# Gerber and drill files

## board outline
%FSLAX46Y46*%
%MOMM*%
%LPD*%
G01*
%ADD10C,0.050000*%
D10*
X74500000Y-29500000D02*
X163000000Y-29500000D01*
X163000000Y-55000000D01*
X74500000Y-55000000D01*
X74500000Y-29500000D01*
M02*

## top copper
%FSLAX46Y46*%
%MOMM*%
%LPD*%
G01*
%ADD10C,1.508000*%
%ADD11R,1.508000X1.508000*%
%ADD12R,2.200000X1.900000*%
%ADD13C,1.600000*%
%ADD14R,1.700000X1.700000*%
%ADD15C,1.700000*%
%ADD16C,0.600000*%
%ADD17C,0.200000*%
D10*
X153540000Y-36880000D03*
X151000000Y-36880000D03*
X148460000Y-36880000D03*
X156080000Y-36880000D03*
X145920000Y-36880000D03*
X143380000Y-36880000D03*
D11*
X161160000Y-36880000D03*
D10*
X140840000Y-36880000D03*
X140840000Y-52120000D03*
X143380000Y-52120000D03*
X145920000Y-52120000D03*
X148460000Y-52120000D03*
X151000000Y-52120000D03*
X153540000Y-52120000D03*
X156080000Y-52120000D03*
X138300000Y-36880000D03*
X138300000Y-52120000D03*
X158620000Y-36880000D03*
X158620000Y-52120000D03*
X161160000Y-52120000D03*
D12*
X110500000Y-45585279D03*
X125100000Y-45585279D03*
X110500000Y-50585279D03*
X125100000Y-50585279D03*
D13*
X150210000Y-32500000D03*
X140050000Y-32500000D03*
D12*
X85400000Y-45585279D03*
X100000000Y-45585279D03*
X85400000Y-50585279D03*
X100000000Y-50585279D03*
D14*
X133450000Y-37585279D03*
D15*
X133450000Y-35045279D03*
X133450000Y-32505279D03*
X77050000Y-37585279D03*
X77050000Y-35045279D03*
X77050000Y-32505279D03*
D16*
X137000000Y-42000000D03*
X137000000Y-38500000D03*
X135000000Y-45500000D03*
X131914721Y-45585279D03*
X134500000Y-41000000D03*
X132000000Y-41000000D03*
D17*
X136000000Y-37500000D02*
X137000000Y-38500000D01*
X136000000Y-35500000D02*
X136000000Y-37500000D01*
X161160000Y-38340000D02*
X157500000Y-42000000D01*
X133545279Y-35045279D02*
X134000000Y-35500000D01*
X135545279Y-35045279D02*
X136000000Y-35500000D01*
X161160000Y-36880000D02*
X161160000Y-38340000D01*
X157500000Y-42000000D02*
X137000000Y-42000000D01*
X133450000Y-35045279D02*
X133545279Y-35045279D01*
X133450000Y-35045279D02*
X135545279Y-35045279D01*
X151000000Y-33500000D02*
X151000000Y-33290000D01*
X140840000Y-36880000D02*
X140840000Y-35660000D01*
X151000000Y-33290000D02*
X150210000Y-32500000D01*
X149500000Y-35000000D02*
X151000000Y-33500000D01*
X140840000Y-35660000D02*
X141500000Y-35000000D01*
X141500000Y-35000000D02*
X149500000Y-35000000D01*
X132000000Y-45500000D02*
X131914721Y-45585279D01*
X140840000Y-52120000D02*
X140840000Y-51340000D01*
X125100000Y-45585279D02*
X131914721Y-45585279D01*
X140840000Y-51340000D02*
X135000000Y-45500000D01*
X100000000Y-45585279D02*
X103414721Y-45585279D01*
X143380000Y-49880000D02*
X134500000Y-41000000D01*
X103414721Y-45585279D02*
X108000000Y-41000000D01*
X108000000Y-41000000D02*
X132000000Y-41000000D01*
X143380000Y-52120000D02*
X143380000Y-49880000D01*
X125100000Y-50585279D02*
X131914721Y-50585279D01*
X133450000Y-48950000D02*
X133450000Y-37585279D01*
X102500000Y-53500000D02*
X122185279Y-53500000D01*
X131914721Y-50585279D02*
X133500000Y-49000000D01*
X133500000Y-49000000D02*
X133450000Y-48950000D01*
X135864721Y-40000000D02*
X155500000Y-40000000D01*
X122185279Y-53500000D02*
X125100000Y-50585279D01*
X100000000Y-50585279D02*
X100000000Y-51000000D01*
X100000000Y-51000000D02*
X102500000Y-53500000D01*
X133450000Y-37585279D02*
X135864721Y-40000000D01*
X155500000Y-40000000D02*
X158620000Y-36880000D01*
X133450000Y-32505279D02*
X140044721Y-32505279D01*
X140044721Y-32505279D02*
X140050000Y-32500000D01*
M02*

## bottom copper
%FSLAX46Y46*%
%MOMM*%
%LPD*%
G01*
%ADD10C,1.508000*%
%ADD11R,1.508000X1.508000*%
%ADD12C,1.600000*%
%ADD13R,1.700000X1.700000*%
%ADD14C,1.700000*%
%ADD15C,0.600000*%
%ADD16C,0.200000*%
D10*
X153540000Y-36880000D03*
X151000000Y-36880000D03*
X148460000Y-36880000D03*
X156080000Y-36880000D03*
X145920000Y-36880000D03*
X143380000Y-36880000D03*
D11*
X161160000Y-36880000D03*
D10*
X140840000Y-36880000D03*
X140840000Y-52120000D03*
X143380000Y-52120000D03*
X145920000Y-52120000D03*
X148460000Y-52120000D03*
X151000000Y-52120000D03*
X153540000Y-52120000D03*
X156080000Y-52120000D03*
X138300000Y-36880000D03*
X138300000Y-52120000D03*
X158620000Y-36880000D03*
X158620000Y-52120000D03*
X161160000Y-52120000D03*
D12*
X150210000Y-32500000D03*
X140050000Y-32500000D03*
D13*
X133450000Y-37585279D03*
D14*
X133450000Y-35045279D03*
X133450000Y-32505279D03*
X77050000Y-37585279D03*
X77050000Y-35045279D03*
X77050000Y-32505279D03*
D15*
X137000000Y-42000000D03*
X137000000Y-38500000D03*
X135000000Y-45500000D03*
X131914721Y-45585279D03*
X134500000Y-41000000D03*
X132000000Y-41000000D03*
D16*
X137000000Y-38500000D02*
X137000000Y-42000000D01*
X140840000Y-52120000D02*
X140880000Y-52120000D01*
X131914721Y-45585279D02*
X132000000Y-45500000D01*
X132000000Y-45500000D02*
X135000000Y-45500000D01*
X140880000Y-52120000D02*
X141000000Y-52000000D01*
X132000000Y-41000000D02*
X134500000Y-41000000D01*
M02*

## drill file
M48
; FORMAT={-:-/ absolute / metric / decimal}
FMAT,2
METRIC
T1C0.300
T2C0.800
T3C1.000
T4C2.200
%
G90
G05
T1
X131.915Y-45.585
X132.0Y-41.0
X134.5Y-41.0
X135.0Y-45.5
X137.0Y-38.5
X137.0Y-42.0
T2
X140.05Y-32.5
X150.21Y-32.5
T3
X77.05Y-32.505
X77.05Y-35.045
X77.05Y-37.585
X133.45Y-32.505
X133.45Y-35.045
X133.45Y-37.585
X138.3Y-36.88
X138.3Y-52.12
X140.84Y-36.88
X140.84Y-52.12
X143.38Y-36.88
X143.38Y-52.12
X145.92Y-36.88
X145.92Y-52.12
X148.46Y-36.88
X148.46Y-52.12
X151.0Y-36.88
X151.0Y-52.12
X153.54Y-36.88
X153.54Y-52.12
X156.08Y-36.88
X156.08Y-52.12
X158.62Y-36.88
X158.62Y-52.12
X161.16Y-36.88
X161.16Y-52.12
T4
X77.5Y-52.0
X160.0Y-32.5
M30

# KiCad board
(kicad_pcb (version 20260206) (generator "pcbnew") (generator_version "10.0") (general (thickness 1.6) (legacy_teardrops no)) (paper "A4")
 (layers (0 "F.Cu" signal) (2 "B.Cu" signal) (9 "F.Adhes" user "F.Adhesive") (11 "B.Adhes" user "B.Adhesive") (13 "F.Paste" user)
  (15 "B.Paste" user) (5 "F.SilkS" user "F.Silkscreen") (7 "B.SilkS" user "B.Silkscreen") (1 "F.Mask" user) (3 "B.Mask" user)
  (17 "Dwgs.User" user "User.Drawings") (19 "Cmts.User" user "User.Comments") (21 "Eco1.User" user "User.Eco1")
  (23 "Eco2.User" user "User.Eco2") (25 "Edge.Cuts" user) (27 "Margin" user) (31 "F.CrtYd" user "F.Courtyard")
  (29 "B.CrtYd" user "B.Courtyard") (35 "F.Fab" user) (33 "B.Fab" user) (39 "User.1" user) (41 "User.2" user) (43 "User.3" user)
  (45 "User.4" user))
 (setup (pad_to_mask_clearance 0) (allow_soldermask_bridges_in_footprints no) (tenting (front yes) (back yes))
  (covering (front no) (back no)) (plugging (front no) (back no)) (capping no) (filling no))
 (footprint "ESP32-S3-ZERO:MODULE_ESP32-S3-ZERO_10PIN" (layer "F.Cu") (at 151 44.5 -90)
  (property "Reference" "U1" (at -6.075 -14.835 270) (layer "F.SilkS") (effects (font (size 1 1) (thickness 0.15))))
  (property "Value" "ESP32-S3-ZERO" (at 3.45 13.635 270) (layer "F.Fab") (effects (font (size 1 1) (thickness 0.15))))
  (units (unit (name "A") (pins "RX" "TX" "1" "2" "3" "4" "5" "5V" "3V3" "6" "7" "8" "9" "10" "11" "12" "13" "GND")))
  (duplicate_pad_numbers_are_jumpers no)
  (pad "1" thru_hole circle (at -7.62 -2.54 270) (size 1.508 1.508) (drill 1) (layers "*.Cu" "*.Mask") (remove_unused_layers no)
   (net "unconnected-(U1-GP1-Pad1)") (solder_mask_margin 0.102))
  (pad "2" thru_hole circle (at -7.62 0 270) (size 1.508 1.508) (drill 1) (layers "*.Cu" "*.Mask") (remove_unused_layers no)
   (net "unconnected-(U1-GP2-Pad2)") (solder_mask_margin 0.102))
  (pad "3" thru_hole circle (at -7.62 2.54 270) (size 1.508 1.508) (drill 1) (layers "*.Cu" "*.Mask") (remove_unused_layers no)
   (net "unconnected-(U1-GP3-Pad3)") (solder_mask_margin 0.102))
  (pad "3V3" thru_hole circle (at -7.62 -5.08 270) (size 1.508 1.508) (drill 1) (layers "*.Cu" "*.Mask") (remove_unused_layers no)
   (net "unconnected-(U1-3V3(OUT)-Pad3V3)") (solder_mask_margin 0.102))
  (pad "4" thru_hole circle (at -7.62 5.08 270) (size 1.508 1.508) (drill 1) (layers "*.Cu" "*.Mask") (remove_unused_layers no)
   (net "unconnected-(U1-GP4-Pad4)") (solder_mask_margin 0.102))
  (pad "5" thru_hole circle (at -7.62 7.62 270) (size 1.508 1.508) (drill 1) (layers "*.Cu" "*.Mask") (remove_unused_layers no)
   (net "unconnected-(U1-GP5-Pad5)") (solder_mask_margin 0.102))
  (pad "5V" thru_hole rect (at -7.62 -10.16 270) (size 1.508 1.508) (drill 1) (layers "*.Cu" "*.Mask") (remove_unused_layers no)
   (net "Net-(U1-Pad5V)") (solder_mask_margin 0.102))
  (pad "6" thru_hole circle (at -7.62 10.16 270) (size 1.508 1.508) (drill 1) (layers "*.Cu" "*.Mask") (remove_unused_layers no)
   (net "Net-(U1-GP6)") (solder_mask_margin 0.102))
  (pad "7" thru_hole circle (at 7.62 10.16 270) (size 1.508 1.508) (drill 1) (layers "*.Cu" "*.Mask") (remove_unused_layers no)
   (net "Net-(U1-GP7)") (solder_mask_margin 0.102))
  (pad "8" thru_hole circle (at 7.62 7.62 270) (size 1.508 1.508) (drill 1) (layers "*.Cu" "*.Mask") (remove_unused_layers no)
   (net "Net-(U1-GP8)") (solder_mask_margin 0.102))
  (pad "9" thru_hole circle (at 7.62 5.08 270) (size 1.508 1.508) (drill 1) (layers "*.Cu" "*.Mask") (remove_unused_layers no)
   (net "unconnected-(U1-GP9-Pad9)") (solder_mask_margin 0.102))
  (pad "10" thru_hole circle (at 7.62 2.54 270) (size 1.508 1.508) (drill 1) (layers "*.Cu" "*.Mask") (remove_unused_layers no)
   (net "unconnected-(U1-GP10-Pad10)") (solder_mask_margin 0.102))
  (pad "11" thru_hole circle (at 7.62 0 270) (size 1.508 1.508) (drill 1) (layers "*.Cu" "*.Mask") (remove_unused_layers no)
   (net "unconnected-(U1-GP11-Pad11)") (solder_mask_margin 0.102))
  (pad "12" thru_hole circle (at 7.62 -2.54 270) (size 1.508 1.508) (drill 1) (layers "*.Cu" "*.Mask") (remove_unused_layers no)
   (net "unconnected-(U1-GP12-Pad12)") (solder_mask_margin 0.102))
  (pad "13" thru_hole circle (at 7.62 -5.08 270) (size 1.508 1.508) (drill 1) (layers "*.Cu" "*.Mask") (remove_unused_layers no)
   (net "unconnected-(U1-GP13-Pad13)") (solder_mask_margin 0.102))
  (pad "14" thru_hole circle (at -7.62 12.7 270) (size 1.508 1.508) (drill 1) (layers "*.Cu" "*.Mask") (remove_unused_layers no)
   (solder_mask_margin 0.102))
  (pad "15" thru_hole circle (at 7.62 12.7 270) (size 1.508 1.508) (drill 1) (layers "*.Cu" "*.Mask") (remove_unused_layers no)
   (solder_mask_margin 0.102))
  (pad "GND" thru_hole circle (at -7.62 -7.62 270) (size 1.508 1.508) (drill 1) (layers "*.Cu" "*.Mask") (remove_unused_layers no)
   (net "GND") (solder_mask_margin 0.102))
  (pad "RX" thru_hole circle (at 7.62 -7.62 270) (size 1.508 1.508) (drill 1) (layers "*.Cu" "*.Mask") (remove_unused_layers no)
   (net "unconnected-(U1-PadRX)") (solder_mask_margin 0.102))
  (pad "TX" thru_hole circle (at 7.62 -10.16 270) (size 1.508 1.508) (drill 1) (layers "*.Cu" "*.Mask") (remove_unused_layers no)
   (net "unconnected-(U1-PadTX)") (solder_mask_margin 0.102)))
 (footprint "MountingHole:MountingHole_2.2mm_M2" (layer "F.Cu") (at 77.5 52)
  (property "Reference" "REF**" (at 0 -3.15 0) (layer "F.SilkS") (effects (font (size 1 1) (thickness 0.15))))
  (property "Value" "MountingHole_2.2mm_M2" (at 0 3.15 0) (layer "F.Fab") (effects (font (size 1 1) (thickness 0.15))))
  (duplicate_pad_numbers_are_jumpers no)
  (pad "" np_thru_hole circle (at 0 0) (size 2.2 2.2) (drill 2.2) (layers "*.Cu" "*.Mask")))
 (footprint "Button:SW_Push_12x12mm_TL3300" (layer "F.Cu") (at 117.8 48.085279)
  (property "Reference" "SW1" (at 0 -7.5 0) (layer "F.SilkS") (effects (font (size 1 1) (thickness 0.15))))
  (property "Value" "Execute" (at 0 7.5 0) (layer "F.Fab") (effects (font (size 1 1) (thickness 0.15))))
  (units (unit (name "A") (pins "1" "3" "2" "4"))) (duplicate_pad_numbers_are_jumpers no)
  (pad "1" smd rect (at -7.3 -2.5) (size 2.2 1.9) (layers "F.Cu" "F.Mask" "F.Paste") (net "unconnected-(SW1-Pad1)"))
  (pad "2" smd rect (at 7.3 -2.5) (size 2.2 1.9) (layers "F.Cu" "F.Mask" "F.Paste") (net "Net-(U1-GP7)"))
  (pad "3" smd rect (at -7.3 2.5) (size 2.2 1.9) (layers "F.Cu" "F.Mask" "F.Paste") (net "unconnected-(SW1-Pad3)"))
  (pad "4" smd rect (at 7.3 2.5) (size 2.2 1.9) (layers "F.Cu" "F.Mask" "F.Paste") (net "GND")))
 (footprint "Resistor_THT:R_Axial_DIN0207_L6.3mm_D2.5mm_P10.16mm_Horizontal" (layer "F.Cu") (at 150.21 32.5 180)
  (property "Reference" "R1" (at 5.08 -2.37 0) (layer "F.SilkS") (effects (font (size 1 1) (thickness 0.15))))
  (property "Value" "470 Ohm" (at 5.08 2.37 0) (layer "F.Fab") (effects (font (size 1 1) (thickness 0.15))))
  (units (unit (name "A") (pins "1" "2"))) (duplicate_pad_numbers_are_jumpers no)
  (pad "1" thru_hole circle (at 0 0 180) (size 1.6 1.6) (drill 0.8) (layers "*.Cu" "*.Mask") (remove_unused_layers no) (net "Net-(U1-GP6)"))
  (pad "2" thru_hole circle (at 10.16 0 180) (size 1.6 1.6) (drill 0.8) (layers "*.Cu" "*.Mask") (remove_unused_layers no)
   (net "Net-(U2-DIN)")))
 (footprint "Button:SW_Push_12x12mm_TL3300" (layer "F.Cu") (at 92.7 48.085279)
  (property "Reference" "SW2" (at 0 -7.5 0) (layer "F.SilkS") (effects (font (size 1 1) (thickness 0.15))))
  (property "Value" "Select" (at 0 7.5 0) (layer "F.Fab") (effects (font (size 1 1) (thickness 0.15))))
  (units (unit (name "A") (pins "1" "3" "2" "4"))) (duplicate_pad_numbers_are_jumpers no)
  (pad "1" smd rect (at -7.3 -2.5) (size 2.2 1.9) (layers "F.Cu" "F.Mask" "F.Paste") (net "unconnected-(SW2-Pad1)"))
  (pad "2" smd rect (at 7.3 -2.5) (size 2.2 1.9) (layers "F.Cu" "F.Mask" "F.Paste") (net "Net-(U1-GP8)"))
  (pad "3" smd rect (at -7.3 2.5) (size 2.2 1.9) (layers "F.Cu" "F.Mask" "F.Paste") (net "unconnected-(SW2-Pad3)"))
  (pad "4" smd rect (at 7.3 2.5) (size 2.2 1.9) (layers "F.Cu" "F.Mask" "F.Paste") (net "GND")))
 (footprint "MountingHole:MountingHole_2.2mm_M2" (layer "F.Cu") (at 160 32.5)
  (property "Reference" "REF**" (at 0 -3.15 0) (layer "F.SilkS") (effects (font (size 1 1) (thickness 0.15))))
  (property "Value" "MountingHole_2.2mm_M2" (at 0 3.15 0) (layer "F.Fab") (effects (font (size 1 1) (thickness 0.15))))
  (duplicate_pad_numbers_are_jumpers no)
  (pad "" np_thru_hole circle (at 0 0) (size 2.2 2.2) (drill 2.2) (layers "*.Cu" "*.Mask")))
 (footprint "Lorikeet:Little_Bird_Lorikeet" (layer "F.Cu") (at 105.25 35.045279 180)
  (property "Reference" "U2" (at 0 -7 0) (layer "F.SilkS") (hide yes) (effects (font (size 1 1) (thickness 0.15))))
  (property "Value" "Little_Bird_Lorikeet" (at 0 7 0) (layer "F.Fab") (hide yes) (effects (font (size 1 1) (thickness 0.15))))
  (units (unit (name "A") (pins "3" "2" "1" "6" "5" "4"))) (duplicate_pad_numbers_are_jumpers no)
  (pad "1" thru_hole rect (at -28.2 -2.54 180) (size 1.7 1.7) (drill 1) (layers "*.Cu" "*.Mask") (remove_unused_layers no) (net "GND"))
  (pad "2" thru_hole circle (at -28.2 0 180) (size 1.7 1.7) (drill 1) (layers "*.Cu" "*.Mask") (remove_unused_layers no)
   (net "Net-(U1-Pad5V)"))
  (pad "3" thru_hole circle (at -28.2 2.54 180) (size 1.7 1.7) (drill 1) (layers "*.Cu" "*.Mask") (remove_unused_layers no)
   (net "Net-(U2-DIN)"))
  (pad "4" thru_hole circle (at 28.2 -2.54 180) (size 1.7 1.7) (drill 1) (layers "*.Cu" "*.Mask") (remove_unused_layers no)
   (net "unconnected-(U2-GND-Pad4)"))
  (pad "5" thru_hole circle (at 28.2 0 180) (size 1.7 1.7) (drill 1) (layers "*.Cu" "*.Mask") (remove_unused_layers no)
   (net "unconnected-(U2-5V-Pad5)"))
  (pad "6" thru_hole circle (at 28.2 2.54 180) (size 1.7 1.7) (drill 1) (layers "*.Cu" "*.Mask") (remove_unused_layers no)
   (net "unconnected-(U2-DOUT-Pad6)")))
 (gr_rect (start 74.5 29.5) (end 163 55) (stroke (width 0.05) (type default)) (fill no) (layer "Edge.Cuts"))
 (segment (start 136 37.5) (end 137 38.5) (width 0.2) (layer "F.Cu") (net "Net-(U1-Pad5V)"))
 (segment (start 136 35.5) (end 136 37.5) (width 0.2) (layer "F.Cu") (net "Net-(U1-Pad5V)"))
 (segment (start 161.16 38.34) (end 157.5 42) (width 0.2) (layer "F.Cu") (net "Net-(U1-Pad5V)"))
 (segment (start 133.545279 35.045279) (end 134 35.5) (width 0.2) (layer "F.Cu") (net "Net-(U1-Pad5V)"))
 (segment (start 135.545279 35.045279) (end 136 35.5) (width 0.2) (layer "F.Cu") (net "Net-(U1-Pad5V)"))
 (segment (start 161.16 36.88) (end 161.16 38.34) (width 0.2) (layer "F.Cu") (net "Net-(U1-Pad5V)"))
 (segment (start 157.5 42) (end 137 42) (width 0.2) (layer "F.Cu") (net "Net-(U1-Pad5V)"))
 (segment (start 133.45 35.045279) (end 133.545279 35.045279) (width 0.2) (layer "F.Cu") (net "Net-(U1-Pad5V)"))
 (segment (start 133.45 35.045279) (end 135.545279 35.045279) (width 0.2) (layer "F.Cu") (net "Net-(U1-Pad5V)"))
 (via (at 137 42) (size 0.6) (drill 0.3) (layers "F.Cu" "B.Cu") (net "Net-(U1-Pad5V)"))
 (via (at 137 38.5) (size 0.6) (drill 0.3) (layers "F.Cu" "B.Cu") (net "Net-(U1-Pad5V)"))
 (segment (start 137 38.5) (end 137 42) (width 0.2) (layer "B.Cu") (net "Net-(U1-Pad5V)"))
 (segment (start 151 33.5) (end 151 33.29) (width 0.2) (layer "F.Cu") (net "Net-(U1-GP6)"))
 (segment (start 140.84 36.88) (end 140.84 35.66) (width 0.2) (layer "F.Cu") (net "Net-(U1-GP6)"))
 (segment (start 151 33.29) (end 150.21 32.5) (width 0.2) (layer "F.Cu") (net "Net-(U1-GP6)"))
 (segment (start 149.5 35) (end 151 33.5) (width 0.2) (layer "F.Cu") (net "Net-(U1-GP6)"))
 (segment (start 140.84 35.66) (end 141.5 35) (width 0.2) (layer "F.Cu") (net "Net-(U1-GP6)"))
 (segment (start 141.5 35) (end 149.5 35) (width 0.2) (layer "F.Cu") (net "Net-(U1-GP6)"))
 (segment (start 132 45.5) (end 131.914721 45.585279) (width 0.2) (layer "F.Cu") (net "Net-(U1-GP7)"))
 (segment (start 140.84 52.12) (end 140.84 51.34) (width 0.2) (layer "F.Cu") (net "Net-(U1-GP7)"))
 (segment (start 125.1 45.585279) (end 131.914721 45.585279) (width 0.2) (layer "F.Cu") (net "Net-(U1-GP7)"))
 (segment (start 140.84 51.34) (end 135 45.5) (width 0.2) (layer "F.Cu") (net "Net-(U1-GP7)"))
 (via (at 135 45.5) (size 0.6) (drill 0.3) (layers "F.Cu" "B.Cu") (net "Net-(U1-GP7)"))
 (via (at 131.914721 45.585279) (size 0.6) (drill 0.3) (layers "F.Cu" "B.Cu") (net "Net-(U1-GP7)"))
 (segment (start 140.84 52.12) (end 140.88 52.12) (width 0.2) (layer "B.Cu") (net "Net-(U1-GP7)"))
 (segment (start 131.914721 45.585279) (end 132 45.5) (width 0.2) (layer "B.Cu") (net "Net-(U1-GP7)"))
 (segment (start 132 45.5) (end 135 45.5) (width 0.2) (layer "B.Cu") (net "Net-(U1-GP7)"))
 (segment (start 140.88 52.12) (end 141 52) (width 0.2) (layer "B.Cu") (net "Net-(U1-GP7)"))
 (segment (start 100 45.585279) (end 103.414721 45.585279) (width 0.2) (layer "F.Cu") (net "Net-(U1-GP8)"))
 (segment (start 143.38 49.88) (end 134.5 41) (width 0.2) (layer "F.Cu") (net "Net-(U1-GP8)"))
 (segment (start 103.414721 45.585279) (end 108 41) (width 0.2) (layer "F.Cu") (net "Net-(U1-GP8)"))
 (segment (start 108 41) (end 132 41) (width 0.2) (layer "F.Cu") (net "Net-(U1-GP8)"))
 (segment (start 143.38 52.12) (end 143.38 49.88) (width 0.2) (layer "F.Cu") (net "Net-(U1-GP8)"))
 (via (at 134.5 41) (size 0.6) (drill 0.3) (layers "F.Cu" "B.Cu") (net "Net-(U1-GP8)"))
 (via (at 132 41) (size 0.6) (drill 0.3) (layers "F.Cu" "B.Cu") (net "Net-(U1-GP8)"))
 (segment (start 132 41) (end 134.5 41) (width 0.2) (layer "B.Cu") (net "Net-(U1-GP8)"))
 (segment (start 125.1 50.585279) (end 131.914721 50.585279) (width 0.2) (layer "F.Cu") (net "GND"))
 (segment (start 133.45 48.95) (end 133.45 37.585279) (width 0.2) (layer "F.Cu") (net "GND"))
 (segment (start 102.5 53.5) (end 122.185279 53.5) (width 0.2) (layer "F.Cu") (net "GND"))
 (segment (start 131.914721 50.585279) (end 133.5 49) (width 0.2) (layer "F.Cu") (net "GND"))
 (segment (start 133.5 49) (end 133.45 48.95) (width 0.2) (layer "F.Cu") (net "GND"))
 (segment (start 135.864721 40) (end 155.5 40) (width 0.2) (layer "F.Cu") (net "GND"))
 (segment (start 122.185279 53.5) (end 125.1 50.585279) (width 0.2) (layer "F.Cu") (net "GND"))
 (segment (start 100 50.585279) (end 100 51) (width 0.2) (layer "F.Cu") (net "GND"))
 (segment (start 100 51) (end 102.5 53.5) (width 0.2) (layer "F.Cu") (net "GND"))
 (segment (start 133.45 37.585279) (end 135.864721 40) (width 0.2) (layer "F.Cu") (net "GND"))
 (segment (start 155.5 40) (end 158.62 36.88) (width 0.2) (layer "F.Cu") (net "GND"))
 (segment (start 133.45 32.505279) (end 140.044721 32.505279) (width 0.2) (layer "F.Cu") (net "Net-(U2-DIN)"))
 (segment (start 140.044721 32.505279) (end 140.05 32.5) (width 0.2) (layer "F.Cu") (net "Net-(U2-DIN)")))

